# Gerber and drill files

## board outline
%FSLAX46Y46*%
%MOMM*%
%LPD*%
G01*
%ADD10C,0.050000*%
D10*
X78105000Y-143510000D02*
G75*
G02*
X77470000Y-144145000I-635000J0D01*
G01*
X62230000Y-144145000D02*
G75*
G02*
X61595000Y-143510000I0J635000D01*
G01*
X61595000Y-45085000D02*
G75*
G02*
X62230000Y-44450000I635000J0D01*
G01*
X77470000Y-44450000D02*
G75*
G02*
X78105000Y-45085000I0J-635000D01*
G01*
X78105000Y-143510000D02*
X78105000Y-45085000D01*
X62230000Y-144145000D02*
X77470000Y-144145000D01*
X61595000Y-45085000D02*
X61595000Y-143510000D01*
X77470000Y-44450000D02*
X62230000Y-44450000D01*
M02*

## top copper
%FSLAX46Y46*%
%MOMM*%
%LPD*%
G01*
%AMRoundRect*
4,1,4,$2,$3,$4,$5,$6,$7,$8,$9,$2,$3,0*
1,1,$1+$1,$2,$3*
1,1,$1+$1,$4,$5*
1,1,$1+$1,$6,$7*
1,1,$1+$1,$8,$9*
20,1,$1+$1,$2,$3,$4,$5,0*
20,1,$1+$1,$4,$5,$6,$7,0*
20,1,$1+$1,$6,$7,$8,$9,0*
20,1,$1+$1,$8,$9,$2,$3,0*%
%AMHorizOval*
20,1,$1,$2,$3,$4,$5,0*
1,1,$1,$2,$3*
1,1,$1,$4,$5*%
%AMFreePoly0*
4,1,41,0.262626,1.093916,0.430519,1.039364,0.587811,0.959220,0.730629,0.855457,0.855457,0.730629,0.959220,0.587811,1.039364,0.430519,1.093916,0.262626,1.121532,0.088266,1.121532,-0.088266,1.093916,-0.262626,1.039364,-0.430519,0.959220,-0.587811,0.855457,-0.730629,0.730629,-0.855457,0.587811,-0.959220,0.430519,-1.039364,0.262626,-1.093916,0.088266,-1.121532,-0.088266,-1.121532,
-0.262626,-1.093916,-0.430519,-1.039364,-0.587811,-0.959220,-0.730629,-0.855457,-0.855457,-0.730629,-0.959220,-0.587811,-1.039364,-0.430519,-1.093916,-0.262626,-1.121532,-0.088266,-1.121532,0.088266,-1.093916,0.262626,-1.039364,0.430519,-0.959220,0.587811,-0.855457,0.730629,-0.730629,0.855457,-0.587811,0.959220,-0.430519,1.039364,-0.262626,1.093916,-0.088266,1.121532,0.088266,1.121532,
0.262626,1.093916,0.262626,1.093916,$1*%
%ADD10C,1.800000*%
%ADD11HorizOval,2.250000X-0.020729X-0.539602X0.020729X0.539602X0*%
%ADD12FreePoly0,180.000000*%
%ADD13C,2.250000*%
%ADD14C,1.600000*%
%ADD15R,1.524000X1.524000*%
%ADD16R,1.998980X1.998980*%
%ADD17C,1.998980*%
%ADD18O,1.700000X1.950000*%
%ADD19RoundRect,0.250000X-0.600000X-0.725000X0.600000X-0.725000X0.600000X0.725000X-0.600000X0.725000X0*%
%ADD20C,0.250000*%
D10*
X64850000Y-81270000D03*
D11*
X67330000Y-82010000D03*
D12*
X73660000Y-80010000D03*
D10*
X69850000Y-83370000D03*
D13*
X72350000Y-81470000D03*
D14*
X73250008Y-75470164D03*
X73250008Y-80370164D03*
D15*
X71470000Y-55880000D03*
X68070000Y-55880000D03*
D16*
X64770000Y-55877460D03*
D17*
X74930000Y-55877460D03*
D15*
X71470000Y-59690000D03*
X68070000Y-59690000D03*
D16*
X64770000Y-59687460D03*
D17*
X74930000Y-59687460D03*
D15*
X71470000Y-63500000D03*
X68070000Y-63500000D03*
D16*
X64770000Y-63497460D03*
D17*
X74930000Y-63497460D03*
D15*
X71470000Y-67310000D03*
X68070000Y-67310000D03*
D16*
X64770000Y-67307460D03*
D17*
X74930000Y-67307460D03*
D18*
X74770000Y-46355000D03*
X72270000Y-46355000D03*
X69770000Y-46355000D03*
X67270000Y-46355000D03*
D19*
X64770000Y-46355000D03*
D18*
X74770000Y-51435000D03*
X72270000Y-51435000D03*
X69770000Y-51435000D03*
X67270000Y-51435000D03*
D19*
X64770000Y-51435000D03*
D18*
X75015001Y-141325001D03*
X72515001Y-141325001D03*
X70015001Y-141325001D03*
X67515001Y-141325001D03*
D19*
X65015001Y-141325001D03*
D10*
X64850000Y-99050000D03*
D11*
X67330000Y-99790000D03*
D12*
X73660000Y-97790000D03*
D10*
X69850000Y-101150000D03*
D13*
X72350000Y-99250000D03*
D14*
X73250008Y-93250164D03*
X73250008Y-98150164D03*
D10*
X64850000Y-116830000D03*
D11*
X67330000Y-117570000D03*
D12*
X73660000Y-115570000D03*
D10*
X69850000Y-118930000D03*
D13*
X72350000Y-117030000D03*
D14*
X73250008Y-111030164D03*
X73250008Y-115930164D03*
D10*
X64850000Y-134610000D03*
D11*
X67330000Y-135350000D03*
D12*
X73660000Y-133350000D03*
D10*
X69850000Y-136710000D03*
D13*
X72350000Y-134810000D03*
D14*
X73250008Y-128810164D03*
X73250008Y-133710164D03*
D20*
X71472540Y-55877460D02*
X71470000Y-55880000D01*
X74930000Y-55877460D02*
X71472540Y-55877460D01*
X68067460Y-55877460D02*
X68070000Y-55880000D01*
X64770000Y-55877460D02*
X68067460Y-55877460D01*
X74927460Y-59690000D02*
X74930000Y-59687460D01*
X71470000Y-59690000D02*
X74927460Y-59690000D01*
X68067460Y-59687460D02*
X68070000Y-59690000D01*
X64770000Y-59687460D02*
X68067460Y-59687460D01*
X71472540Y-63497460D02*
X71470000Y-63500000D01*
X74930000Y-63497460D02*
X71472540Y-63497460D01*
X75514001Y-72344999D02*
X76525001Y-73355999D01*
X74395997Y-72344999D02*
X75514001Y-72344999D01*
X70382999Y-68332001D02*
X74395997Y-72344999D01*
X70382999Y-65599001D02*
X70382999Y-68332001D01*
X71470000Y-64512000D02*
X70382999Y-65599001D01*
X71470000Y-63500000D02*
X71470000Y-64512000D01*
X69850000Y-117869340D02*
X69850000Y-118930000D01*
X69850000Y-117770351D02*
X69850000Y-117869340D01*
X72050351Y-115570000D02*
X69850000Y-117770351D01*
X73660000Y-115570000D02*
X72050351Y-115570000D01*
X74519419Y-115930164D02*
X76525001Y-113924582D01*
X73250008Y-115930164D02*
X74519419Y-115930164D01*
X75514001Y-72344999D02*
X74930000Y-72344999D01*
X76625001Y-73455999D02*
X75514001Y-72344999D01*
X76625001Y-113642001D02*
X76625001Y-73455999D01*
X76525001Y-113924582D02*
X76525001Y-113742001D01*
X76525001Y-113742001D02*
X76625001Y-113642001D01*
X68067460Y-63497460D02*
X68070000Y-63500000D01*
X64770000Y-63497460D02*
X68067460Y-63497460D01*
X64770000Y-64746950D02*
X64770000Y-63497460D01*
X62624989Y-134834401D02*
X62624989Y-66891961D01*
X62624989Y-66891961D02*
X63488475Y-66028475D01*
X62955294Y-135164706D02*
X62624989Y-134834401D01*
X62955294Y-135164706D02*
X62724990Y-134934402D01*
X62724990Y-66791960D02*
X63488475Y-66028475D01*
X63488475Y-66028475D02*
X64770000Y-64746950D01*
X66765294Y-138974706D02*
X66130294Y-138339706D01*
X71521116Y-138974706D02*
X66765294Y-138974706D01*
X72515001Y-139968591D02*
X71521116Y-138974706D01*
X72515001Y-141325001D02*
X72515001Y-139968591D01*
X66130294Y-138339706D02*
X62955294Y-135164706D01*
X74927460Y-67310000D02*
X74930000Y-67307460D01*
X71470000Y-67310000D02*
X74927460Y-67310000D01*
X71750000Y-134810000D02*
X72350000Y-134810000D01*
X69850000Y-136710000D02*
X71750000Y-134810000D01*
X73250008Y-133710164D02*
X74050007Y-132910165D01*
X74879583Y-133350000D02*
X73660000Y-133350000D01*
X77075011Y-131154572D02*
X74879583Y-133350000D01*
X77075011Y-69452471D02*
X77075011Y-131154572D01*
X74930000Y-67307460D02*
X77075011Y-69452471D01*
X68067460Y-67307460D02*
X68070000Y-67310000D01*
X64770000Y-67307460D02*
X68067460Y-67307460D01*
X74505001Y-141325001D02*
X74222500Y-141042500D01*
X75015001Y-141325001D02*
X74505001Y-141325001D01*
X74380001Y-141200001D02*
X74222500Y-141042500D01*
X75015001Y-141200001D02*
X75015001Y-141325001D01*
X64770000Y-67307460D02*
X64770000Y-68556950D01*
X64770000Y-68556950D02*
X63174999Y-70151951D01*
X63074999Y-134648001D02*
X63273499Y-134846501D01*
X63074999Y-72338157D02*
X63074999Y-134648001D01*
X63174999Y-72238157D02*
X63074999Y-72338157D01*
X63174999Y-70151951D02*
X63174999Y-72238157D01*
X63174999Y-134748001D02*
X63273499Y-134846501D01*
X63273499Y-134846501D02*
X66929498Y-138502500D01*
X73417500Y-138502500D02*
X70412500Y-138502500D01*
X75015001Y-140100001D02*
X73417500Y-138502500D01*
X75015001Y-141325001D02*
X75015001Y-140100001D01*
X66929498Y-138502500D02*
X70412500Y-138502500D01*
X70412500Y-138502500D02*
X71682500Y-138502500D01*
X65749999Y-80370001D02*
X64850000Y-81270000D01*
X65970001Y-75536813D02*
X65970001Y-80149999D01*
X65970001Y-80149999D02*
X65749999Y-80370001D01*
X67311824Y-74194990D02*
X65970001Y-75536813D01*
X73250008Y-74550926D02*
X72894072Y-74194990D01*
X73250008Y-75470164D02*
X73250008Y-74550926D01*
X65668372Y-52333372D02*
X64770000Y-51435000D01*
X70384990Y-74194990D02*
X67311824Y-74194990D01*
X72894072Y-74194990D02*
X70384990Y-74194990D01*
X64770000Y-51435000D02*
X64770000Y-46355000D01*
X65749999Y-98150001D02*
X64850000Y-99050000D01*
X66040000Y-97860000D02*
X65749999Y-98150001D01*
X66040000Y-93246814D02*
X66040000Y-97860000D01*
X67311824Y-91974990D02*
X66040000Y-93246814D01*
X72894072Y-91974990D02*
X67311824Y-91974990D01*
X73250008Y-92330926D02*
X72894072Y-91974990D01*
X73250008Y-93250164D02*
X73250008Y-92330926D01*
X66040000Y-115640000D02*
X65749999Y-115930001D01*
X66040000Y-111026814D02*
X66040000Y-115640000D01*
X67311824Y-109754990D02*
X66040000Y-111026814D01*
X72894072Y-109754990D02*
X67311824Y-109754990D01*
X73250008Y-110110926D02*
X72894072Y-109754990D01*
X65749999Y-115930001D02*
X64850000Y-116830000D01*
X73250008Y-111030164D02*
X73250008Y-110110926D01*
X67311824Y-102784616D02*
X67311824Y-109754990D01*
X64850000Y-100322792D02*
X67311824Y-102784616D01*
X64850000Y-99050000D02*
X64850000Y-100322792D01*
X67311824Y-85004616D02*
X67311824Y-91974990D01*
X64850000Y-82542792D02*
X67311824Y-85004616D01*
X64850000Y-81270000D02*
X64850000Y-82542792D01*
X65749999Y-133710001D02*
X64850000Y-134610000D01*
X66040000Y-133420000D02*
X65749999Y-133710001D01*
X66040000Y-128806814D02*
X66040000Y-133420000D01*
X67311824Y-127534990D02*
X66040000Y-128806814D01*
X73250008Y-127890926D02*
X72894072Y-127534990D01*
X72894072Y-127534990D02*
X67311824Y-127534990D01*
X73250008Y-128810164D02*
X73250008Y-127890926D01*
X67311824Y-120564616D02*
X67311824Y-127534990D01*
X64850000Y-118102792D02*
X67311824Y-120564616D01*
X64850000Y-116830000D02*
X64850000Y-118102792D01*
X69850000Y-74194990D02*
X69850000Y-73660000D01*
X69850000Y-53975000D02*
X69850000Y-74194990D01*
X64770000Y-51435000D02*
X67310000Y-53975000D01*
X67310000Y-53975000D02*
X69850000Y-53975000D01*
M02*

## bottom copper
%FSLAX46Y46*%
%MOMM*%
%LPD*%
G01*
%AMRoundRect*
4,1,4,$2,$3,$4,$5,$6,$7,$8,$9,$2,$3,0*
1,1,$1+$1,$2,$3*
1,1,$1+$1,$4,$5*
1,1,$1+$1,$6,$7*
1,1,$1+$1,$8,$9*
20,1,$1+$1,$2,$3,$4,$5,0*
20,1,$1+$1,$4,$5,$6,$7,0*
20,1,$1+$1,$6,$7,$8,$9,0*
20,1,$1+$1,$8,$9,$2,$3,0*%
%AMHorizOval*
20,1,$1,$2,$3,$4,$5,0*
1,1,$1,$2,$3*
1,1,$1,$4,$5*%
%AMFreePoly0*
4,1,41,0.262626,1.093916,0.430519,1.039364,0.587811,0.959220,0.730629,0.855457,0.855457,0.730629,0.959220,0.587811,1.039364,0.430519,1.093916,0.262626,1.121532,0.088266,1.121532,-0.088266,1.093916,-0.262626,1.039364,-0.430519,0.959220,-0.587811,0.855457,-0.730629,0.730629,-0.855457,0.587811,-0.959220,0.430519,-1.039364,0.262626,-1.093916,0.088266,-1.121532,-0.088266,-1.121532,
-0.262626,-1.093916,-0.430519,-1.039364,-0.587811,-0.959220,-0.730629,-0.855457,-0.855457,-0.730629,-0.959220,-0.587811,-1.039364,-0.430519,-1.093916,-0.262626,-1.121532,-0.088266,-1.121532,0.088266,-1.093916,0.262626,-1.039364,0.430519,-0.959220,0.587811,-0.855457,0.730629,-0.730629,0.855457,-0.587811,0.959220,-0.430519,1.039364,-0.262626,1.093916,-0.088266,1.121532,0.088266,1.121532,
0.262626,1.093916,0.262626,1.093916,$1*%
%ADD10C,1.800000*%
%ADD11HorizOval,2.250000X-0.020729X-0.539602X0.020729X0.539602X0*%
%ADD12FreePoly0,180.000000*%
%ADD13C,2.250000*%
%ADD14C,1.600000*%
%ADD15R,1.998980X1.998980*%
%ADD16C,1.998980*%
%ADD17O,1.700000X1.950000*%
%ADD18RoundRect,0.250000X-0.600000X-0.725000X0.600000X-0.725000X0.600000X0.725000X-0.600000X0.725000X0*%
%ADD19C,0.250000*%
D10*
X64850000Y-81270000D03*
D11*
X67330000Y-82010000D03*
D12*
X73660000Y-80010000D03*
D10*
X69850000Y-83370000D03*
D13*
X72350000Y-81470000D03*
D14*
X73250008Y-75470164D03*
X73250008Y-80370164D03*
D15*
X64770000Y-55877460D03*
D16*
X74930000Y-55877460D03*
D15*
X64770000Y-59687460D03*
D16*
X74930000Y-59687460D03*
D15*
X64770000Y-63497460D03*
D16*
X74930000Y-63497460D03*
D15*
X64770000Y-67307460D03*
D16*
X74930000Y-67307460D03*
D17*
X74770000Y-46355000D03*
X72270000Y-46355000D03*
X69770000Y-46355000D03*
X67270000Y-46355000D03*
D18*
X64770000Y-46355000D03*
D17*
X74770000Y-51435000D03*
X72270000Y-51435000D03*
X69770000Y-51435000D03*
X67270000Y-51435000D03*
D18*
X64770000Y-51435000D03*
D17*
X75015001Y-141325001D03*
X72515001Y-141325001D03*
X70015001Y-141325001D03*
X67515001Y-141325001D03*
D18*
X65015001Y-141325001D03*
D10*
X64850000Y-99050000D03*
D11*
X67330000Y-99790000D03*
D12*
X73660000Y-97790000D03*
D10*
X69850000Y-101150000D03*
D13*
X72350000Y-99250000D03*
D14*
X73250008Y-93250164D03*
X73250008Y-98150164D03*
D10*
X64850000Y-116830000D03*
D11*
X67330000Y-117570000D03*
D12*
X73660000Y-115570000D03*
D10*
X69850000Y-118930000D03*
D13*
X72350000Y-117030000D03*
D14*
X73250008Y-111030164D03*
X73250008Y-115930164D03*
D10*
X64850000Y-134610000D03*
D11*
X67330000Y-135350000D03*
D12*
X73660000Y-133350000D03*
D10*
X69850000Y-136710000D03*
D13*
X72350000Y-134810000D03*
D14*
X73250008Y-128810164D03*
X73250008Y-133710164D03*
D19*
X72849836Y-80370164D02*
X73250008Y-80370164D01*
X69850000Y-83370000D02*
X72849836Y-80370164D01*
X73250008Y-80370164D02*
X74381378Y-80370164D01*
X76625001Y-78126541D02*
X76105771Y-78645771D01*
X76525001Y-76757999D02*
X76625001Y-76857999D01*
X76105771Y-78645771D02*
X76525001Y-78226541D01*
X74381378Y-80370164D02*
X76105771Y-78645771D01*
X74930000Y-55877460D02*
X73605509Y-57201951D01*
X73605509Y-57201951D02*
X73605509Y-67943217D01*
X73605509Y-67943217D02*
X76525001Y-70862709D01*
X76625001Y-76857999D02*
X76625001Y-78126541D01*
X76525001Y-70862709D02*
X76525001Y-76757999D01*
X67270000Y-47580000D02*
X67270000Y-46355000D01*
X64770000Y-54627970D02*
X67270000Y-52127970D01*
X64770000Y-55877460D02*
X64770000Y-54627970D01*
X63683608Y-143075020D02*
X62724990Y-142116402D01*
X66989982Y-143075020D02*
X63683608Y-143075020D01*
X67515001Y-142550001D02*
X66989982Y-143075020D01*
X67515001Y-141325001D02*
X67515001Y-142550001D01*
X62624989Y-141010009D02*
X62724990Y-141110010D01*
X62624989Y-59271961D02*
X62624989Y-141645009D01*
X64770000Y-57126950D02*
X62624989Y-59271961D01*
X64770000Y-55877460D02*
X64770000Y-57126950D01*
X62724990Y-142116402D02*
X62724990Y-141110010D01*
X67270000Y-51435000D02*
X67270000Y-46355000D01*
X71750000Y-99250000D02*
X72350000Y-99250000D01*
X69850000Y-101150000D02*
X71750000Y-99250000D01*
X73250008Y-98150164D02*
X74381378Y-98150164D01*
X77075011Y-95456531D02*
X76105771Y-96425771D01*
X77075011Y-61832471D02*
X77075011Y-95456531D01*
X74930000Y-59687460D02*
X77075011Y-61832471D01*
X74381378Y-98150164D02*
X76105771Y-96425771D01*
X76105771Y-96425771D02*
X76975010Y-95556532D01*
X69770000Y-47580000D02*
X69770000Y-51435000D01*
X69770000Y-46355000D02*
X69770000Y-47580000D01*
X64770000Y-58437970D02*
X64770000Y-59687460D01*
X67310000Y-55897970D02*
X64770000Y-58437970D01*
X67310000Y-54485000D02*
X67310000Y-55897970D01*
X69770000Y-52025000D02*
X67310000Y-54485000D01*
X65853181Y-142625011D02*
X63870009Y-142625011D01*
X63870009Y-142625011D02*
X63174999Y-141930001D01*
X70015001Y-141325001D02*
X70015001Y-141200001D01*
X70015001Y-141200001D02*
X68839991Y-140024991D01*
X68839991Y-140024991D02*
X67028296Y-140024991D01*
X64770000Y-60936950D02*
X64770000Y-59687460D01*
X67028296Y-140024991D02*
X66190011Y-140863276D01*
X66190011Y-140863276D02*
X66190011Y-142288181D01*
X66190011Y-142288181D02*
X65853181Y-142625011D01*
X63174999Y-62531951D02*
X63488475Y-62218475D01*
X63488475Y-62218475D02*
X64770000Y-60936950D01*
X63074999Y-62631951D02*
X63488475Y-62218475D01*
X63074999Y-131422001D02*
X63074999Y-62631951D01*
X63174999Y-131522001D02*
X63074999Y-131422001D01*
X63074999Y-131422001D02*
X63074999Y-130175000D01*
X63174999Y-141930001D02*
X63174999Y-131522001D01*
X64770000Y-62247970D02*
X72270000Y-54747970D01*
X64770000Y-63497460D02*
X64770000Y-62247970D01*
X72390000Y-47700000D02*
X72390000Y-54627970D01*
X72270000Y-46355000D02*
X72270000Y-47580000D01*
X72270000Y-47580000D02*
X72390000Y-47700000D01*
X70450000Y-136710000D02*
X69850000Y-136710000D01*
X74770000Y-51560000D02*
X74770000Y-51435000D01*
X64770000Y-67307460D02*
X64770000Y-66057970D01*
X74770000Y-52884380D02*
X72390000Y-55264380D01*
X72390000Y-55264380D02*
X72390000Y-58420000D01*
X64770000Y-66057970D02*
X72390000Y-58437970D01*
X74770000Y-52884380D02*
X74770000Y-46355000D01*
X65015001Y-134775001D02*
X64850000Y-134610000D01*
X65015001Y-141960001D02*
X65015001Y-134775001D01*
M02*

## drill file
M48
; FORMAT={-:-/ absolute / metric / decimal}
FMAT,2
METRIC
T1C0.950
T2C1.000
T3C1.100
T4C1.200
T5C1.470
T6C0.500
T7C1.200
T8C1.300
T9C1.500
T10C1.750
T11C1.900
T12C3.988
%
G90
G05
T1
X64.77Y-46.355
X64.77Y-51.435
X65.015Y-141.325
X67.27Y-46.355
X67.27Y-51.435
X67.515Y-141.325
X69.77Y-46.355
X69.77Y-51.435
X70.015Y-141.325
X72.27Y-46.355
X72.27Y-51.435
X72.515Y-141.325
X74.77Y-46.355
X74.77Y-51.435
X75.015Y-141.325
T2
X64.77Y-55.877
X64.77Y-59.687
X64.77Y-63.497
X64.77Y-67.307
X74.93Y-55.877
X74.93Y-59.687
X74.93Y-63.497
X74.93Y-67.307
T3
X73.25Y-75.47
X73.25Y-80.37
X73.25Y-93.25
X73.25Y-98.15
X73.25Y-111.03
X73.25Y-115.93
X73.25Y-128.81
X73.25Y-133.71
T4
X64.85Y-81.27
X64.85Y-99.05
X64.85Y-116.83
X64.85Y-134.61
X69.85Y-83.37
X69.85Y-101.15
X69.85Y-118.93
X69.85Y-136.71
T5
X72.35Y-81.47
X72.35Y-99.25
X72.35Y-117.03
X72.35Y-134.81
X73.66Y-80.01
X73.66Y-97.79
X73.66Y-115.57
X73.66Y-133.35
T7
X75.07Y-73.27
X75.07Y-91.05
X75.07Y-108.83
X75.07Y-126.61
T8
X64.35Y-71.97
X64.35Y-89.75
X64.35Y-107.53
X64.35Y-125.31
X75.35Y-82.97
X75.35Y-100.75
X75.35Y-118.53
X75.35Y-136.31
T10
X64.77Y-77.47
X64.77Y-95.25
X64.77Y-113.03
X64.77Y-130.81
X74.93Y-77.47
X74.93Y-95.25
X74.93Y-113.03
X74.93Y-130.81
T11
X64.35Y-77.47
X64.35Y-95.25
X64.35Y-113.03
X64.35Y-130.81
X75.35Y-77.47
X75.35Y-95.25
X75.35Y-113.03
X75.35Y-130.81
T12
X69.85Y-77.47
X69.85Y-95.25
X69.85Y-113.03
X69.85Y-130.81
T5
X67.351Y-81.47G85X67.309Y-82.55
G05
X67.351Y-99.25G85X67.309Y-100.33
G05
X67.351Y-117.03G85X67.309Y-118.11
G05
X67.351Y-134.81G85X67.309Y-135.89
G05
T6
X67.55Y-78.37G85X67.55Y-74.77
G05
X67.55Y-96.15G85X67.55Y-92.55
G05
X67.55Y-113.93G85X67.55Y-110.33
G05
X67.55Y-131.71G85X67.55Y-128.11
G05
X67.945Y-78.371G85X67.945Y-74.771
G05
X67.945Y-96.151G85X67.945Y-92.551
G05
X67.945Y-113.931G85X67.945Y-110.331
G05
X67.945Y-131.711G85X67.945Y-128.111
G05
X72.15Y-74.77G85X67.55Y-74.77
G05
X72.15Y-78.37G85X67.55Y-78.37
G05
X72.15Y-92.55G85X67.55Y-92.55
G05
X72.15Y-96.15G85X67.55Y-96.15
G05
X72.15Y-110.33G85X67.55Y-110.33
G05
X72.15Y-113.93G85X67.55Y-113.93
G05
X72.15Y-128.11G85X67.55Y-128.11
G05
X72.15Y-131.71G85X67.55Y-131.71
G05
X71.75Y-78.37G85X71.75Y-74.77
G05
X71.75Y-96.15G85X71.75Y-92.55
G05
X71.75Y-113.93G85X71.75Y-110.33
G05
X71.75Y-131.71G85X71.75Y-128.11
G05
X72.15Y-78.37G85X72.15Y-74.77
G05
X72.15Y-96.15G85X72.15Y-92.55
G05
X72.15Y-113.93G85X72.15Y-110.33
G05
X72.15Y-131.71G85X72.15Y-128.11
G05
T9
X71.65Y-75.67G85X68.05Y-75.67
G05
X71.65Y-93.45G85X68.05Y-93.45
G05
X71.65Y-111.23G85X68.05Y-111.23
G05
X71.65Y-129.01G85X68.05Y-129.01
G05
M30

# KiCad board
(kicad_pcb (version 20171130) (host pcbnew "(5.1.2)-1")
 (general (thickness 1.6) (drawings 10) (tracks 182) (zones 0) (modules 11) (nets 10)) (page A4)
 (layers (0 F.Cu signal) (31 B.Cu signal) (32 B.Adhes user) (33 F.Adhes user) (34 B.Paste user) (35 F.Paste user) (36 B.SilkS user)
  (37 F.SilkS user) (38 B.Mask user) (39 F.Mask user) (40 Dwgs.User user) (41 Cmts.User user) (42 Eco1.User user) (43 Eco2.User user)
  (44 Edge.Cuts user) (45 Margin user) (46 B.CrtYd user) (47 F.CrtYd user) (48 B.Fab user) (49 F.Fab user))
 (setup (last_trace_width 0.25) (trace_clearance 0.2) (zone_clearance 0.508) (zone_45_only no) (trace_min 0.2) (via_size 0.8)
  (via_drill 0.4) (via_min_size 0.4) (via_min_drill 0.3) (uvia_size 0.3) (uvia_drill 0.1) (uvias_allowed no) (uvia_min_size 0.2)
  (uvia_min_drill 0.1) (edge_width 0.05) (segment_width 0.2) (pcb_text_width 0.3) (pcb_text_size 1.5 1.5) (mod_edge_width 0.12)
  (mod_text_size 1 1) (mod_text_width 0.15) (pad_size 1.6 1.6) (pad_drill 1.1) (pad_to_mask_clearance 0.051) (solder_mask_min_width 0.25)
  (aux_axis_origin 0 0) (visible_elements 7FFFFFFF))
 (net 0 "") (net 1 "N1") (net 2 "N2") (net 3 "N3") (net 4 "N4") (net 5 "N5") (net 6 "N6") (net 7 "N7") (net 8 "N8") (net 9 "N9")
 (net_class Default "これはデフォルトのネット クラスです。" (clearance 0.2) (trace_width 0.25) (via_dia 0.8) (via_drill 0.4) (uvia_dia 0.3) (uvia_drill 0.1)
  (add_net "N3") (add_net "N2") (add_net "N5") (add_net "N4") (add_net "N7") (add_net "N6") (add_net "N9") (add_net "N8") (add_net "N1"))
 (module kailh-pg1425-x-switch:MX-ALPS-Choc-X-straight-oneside (layer F.Cu) (at 67.31 82.55 180)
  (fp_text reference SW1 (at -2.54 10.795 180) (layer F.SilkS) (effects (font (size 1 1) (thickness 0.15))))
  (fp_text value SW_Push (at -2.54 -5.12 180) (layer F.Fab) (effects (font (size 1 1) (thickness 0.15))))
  (pad "" np_thru_hole circle (at 2.96 5.08 228.1) (size 1.9 1.9) (drill 1.9) (layers *.Cu *.Mask))
  (pad "" np_thru_hole circle (at -8.04 5.08 228.1) (size 1.9 1.9) (drill 1.9) (layers *.Cu *.Mask))
  (pad 1 thru_hole circle (at 2.46 1.28 180) (size 1.8 1.8) (drill 1.2) (layers *.Cu *.Mask) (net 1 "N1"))
  (pad "" np_thru_hole circle (at 2.54 5.08 228.0996) (size 1.75 1.75) (drill 1.75) (layers *.Cu *.Mask))
  (pad "" np_thru_hole circle (at -7.62 5.08 228.0996) (size 1.75 1.75) (drill 1.75) (layers *.Cu *.Mask))
  (pad "" np_thru_hole circle (at -2.54 5.08 180) (size 3.9878 3.9878) (drill 3.9878) (layers *.Cu *.Mask))
  (pad 3 thru_hole oval (at -0.02 0.54 267.8) (size 3.33 2.25) (drill oval 2.55 1.47) (layers *.Cu *.Mask))
  (pad 2 thru_hole custom (at -6.35 2.54 180) (size 2.25 2.25) (drill 1.47) (layers *.Cu *.Mask) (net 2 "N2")
   (options (clearance outline) (anchor circle)) (primitives))
  (pad "" np_thru_hole circle (at -7.76 9.28 228.1) (size 1.2 1.2) (drill 1.2) (layers *.Cu *.Mask))
  (pad "" np_thru_hole oval (at -0.635 5.97916 180) (size 0.5 4.1) (drill oval 0.5 4.1) (layers *.Cu *.Mask))
  (pad "" np_thru_hole oval (at -4.84 5.98 180) (size 0.5 4.1) (drill oval 0.5 4.1) (layers *.Cu *.Mask))
  (pad "" np_thru_hole oval (at -2.54 6.88 180) (size 5.1 1.5) (drill oval 5.1 1.5) (layers *.Cu *.Mask))
  (pad "" np_thru_hole oval (at -4.44 5.98 180) (size 0.5 4.1) (drill oval 0.5 4.1) (layers *.Cu *.Mask))
  (pad "" np_thru_hole oval (at -2.54 7.78 180) (size 5.1 0.5) (drill oval 5.1 0.5) (layers *.Cu *.Mask))
  (pad "" np_thru_hole oval (at -2.54 4.18 180) (size 5.1 0.5) (drill oval 5.1 0.5) (layers *.Cu *.Mask))
  (pad "" np_thru_hole oval (at -0.24 5.98 180) (size 0.5 4.1) (drill oval 0.5 4.1) (layers *.Cu *.Mask))
  (pad 2 thru_hole circle (at -2.54 -0.82 180) (size 1.8 1.8) (drill 1.2) (layers *.Cu *.Mask) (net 2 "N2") (zone_connect 0))
  (pad 2 thru_hole circle (at -5.04 1.08 180) (size 2.25 2.25) (drill 1.47) (layers *.Cu B.Mask) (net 2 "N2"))
  (pad "" np_thru_hole circle (at 2.959992 10.579836) (size 1.3 1.3) (drill 1.3) (layers *.Cu *.Mask))
  (pad 1 thru_hole circle (at -5.940008 7.079836) (size 1.6 1.6) (drill 1.1) (layers *.Cu *.Mask) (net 1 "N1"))
  (pad "" np_thru_hole circle (at -8.040008 -0.420164) (size 1.3 1.3) (drill 1.3) (layers *.Cu *.Mask))
  (pad 2 thru_hole circle (at -5.940008 2.179836) (size 1.6 1.6) (drill 1.1) (layers *.Cu *.Mask) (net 2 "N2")))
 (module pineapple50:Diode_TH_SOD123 (layer F.Cu) (at 64.77 55.88)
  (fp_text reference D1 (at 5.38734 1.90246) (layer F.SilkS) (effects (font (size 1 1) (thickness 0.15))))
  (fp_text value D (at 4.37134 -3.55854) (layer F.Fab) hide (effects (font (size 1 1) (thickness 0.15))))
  (pad 2 smd rect (at 6.7 0) (size 1.524 1.524) (layers F.Cu F.Paste F.Mask) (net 2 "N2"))
  (pad 1 smd rect (at 3.3 0) (size 1.524 1.524) (layers F.Cu F.Paste F.Mask) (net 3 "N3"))
  (pad 1 thru_hole rect (at 0 -0.00254 180) (size 1.99898 1.99898) (drill 1) (layers *.Cu *.Mask) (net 3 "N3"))
  (pad 2 thru_hole circle (at 10.16 -0.00254 180) (size 1.99898 1.99898) (drill 1) (layers *.Cu *.Mask) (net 2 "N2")))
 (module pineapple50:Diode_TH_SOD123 (layer F.Cu) (at 64.77 59.69)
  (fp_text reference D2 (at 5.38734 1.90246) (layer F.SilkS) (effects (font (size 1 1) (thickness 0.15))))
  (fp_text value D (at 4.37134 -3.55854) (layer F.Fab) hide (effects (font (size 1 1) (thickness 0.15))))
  (pad 2 smd rect (at 6.7 0) (size 1.524 1.524) (layers F.Cu F.Paste F.Mask) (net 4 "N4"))
  (pad 1 smd rect (at 3.3 0) (size 1.524 1.524) (layers F.Cu F.Paste F.Mask) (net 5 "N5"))
  (pad 1 thru_hole rect (at 0 -0.00254 180) (size 1.99898 1.99898) (drill 1) (layers *.Cu *.Mask) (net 5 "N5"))
  (pad 2 thru_hole circle (at 10.16 -0.00254 180) (size 1.99898 1.99898) (drill 1) (layers *.Cu *.Mask) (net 4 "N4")))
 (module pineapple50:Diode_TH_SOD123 (layer F.Cu) (at 64.77 63.5)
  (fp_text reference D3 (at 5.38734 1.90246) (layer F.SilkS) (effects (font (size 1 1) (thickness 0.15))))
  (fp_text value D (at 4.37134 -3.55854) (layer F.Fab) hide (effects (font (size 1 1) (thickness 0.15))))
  (pad 2 smd rect (at 6.7 0) (size 1.524 1.524) (layers F.Cu F.Paste F.Mask) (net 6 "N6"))
  (pad 1 smd rect (at 3.3 0) (size 1.524 1.524) (layers F.Cu F.Paste F.Mask) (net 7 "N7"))
  (pad 1 thru_hole rect (at 0 -0.00254 180) (size 1.99898 1.99898) (drill 1) (layers *.Cu *.Mask) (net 7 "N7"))
  (pad 2 thru_hole circle (at 10.16 -0.00254 180) (size 1.99898 1.99898) (drill 1) (layers *.Cu *.Mask) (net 6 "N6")))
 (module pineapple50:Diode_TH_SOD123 (layer F.Cu) (at 64.77 67.31)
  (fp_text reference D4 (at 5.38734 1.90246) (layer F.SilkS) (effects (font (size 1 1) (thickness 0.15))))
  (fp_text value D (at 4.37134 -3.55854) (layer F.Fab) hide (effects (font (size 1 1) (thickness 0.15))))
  (pad 2 smd rect (at 6.7 0) (size 1.524 1.524) (layers F.Cu F.Paste F.Mask) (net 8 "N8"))
  (pad 1 smd rect (at 3.3 0) (size 1.524 1.524) (layers F.Cu F.Paste F.Mask) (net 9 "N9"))
  (pad 1 thru_hole rect (at 0 -0.00254 180) (size 1.99898 1.99898) (drill 1) (layers *.Cu *.Mask) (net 9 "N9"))
  (pad 2 thru_hole circle (at 10.16 -0.00254 180) (size 1.99898 1.99898) (drill 1) (layers *.Cu *.Mask) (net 8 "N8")))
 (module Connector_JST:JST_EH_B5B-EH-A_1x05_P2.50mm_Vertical (layer F.Cu) (at 64.77 46.355)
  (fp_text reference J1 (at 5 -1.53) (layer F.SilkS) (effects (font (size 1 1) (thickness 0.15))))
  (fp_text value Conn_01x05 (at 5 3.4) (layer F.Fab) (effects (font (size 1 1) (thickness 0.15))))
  (pad 5 thru_hole oval (at 10 0) (size 1.7 1.95) (drill 0.95) (layers *.Cu *.Mask) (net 9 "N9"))
  (pad 4 thru_hole oval (at 7.5 0) (size 1.7 1.95) (drill 0.95) (layers *.Cu *.Mask) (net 7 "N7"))
  (pad 3 thru_hole oval (at 5 0) (size 1.7 1.95) (drill 0.95) (layers *.Cu *.Mask) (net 5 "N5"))
  (pad 2 thru_hole oval (at 2.5 0) (size 1.7 1.95) (drill 0.95) (layers *.Cu *.Mask) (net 3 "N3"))
  (pad 1 thru_hole roundrect (at 0 0) (size 1.7 1.95) (drill 0.95) (layers *.Cu *.Mask) (roundrect_rratio 0.147059) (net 1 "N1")))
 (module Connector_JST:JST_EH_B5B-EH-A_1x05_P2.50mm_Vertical (layer F.Cu) (at 64.77 51.435)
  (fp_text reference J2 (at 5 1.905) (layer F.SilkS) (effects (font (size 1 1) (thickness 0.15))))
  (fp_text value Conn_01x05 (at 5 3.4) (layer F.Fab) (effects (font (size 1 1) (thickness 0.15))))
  (pad 5 thru_hole oval (at 10 0) (size 1.7 1.95) (drill 0.95) (layers *.Cu *.Mask) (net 9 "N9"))
  (pad 4 thru_hole oval (at 7.5 0) (size 1.7 1.95) (drill 0.95) (layers *.Cu *.Mask) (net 7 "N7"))
  (pad 3 thru_hole oval (at 5 0) (size 1.7 1.95) (drill 0.95) (layers *.Cu *.Mask) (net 5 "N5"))
  (pad 2 thru_hole oval (at 2.5 0) (size 1.7 1.95) (drill 0.95) (layers *.Cu *.Mask) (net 3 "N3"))
  (pad 1 thru_hole roundrect (at 0 0) (size 1.7 1.95) (drill 0.95) (layers *.Cu *.Mask) (roundrect_rratio 0.147059) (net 1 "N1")))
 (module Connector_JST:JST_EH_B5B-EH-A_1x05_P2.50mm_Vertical (layer F.Cu) (at 65.015001 141.325001)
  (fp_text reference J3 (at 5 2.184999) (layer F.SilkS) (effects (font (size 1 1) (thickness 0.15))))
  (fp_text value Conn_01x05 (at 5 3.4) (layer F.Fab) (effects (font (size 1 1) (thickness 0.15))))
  (pad 5 thru_hole oval (at 10 0) (size 1.7 1.95) (drill 0.95) (layers *.Cu *.Mask) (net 9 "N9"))
  (pad 4 thru_hole oval (at 7.5 0) (size 1.7 1.95) (drill 0.95) (layers *.Cu *.Mask) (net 7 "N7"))
  (pad 3 thru_hole oval (at 5 0) (size 1.7 1.95) (drill 0.95) (layers *.Cu *.Mask) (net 5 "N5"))
  (pad 2 thru_hole oval (at 2.5 0) (size 1.7 1.95) (drill 0.95) (layers *.Cu *.Mask) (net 3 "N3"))
  (pad 1 thru_hole roundrect (at 0 0) (size 1.7 1.95) (drill 0.95) (layers *.Cu *.Mask) (roundrect_rratio 0.147059) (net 1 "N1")))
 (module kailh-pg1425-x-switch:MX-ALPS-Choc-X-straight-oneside (layer F.Cu) (at 67.31 100.33 180)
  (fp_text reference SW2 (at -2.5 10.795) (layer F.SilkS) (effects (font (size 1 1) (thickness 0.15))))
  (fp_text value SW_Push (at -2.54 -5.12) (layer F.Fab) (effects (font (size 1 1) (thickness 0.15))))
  (pad "" np_thru_hole circle (at 2.96 5.08 228.1) (size 1.9 1.9) (drill 1.9) (layers *.Cu *.Mask))
  (pad "" np_thru_hole circle (at -8.04 5.08 228.1) (size 1.9 1.9) (drill 1.9) (layers *.Cu *.Mask))
  (pad 1 thru_hole circle (at 2.46 1.28 180) (size 1.8 1.8) (drill 1.2) (layers *.Cu *.Mask) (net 1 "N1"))
  (pad "" np_thru_hole circle (at 2.54 5.08 228.0996) (size 1.75 1.75) (drill 1.75) (layers *.Cu *.Mask))
  (pad "" np_thru_hole circle (at -7.62 5.08 228.0996) (size 1.75 1.75) (drill 1.75) (layers *.Cu *.Mask))
  (pad "" np_thru_hole circle (at -2.54 5.08 180) (size 3.9878 3.9878) (drill 3.9878) (layers *.Cu *.Mask))
  (pad 3 thru_hole oval (at -0.02 0.54 267.8) (size 3.33 2.25) (drill oval 2.55 1.47) (layers *.Cu *.Mask))
  (pad 2 thru_hole custom (at -6.35 2.54 180) (size 2.25 2.25) (drill 1.47) (layers *.Cu *.Mask) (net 4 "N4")
   (options (clearance outline) (anchor circle)) (primitives))
  (pad "" np_thru_hole circle (at -7.76 9.28 228.1) (size 1.2 1.2) (drill 1.2) (layers *.Cu *.Mask))
  (pad "" np_thru_hole oval (at -0.635 5.97916 180) (size 0.5 4.1) (drill oval 0.5 4.1) (layers *.Cu *.Mask))
  (pad "" np_thru_hole oval (at -4.84 5.98 180) (size 0.5 4.1) (drill oval 0.5 4.1) (layers *.Cu *.Mask))
  (pad "" np_thru_hole oval (at -2.54 6.88 180) (size 5.1 1.5) (drill oval 5.1 1.5) (layers *.Cu *.Mask))
  (pad "" np_thru_hole oval (at -4.44 5.98 180) (size 0.5 4.1) (drill oval 0.5 4.1) (layers *.Cu *.Mask))
  (pad "" np_thru_hole oval (at -2.54 7.78 180) (size 5.1 0.5) (drill oval 5.1 0.5) (layers *.Cu *.Mask))
  (pad "" np_thru_hole oval (at -2.54 4.18 180) (size 5.1 0.5) (drill oval 5.1 0.5) (layers *.Cu *.Mask))
  (pad "" np_thru_hole oval (at -0.24 5.98 180) (size 0.5 4.1) (drill oval 0.5 4.1) (layers *.Cu *.Mask))
  (pad 2 thru_hole circle (at -2.54 -0.82 180) (size 1.8 1.8) (drill 1.2) (layers *.Cu *.Mask) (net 4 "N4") (zone_connect 0))
  (pad 2 thru_hole circle (at -5.04 1.08 180) (size 2.25 2.25) (drill 1.47) (layers *.Cu B.Mask) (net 4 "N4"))
  (pad "" np_thru_hole circle (at 2.959992 10.579836) (size 1.3 1.3) (drill 1.3) (layers *.Cu *.Mask))
  (pad 1 thru_hole circle (at -5.940008 7.079836) (size 1.6 1.6) (drill 1.1) (layers *.Cu *.Mask) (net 1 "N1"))
  (pad "" np_thru_hole circle (at -8.040008 -0.420164) (size 1.3 1.3) (drill 1.3) (layers *.Cu *.Mask))
  (pad 2 thru_hole circle (at -5.940008 2.179836) (size 1.6 1.6) (drill 1.1) (layers *.Cu *.Mask) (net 4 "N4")))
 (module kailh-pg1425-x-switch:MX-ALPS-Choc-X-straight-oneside (layer F.Cu) (at 67.31 118.11 180)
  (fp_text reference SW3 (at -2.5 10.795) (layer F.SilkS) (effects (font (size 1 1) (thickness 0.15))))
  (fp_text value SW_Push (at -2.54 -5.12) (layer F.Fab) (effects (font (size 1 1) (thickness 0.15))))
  (pad "" np_thru_hole circle (at 2.96 5.08 228.1) (size 1.9 1.9) (drill 1.9) (layers *.Cu *.Mask))
  (pad "" np_thru_hole circle (at -8.04 5.08 228.1) (size 1.9 1.9) (drill 1.9) (layers *.Cu *.Mask))
  (pad 1 thru_hole circle (at 2.46 1.28 180) (size 1.8 1.8) (drill 1.2) (layers *.Cu *.Mask) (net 1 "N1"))
  (pad "" np_thru_hole circle (at 2.54 5.08 228.0996) (size 1.75 1.75) (drill 1.75) (layers *.Cu *.Mask))
  (pad "" np_thru_hole circle (at -7.62 5.08 228.0996) (size 1.75 1.75) (drill 1.75) (layers *.Cu *.Mask))
  (pad "" np_thru_hole circle (at -2.54 5.08 180) (size 3.9878 3.9878) (drill 3.9878) (layers *.Cu *.Mask))
  (pad 3 thru_hole oval (at -0.02 0.54 267.8) (size 3.33 2.25) (drill oval 2.55 1.47) (layers *.Cu *.Mask))
  (pad 2 thru_hole custom (at -6.35 2.54 180) (size 2.25 2.25) (drill 1.47) (layers *.Cu *.Mask) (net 6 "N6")
   (options (clearance outline) (anchor circle)) (primitives))
  (pad "" np_thru_hole circle (at -7.76 9.28 228.1) (size 1.2 1.2) (drill 1.2) (layers *.Cu *.Mask))
  (pad "" np_thru_hole oval (at -0.635 5.97916 180) (size 0.5 4.1) (drill oval 0.5 4.1) (layers *.Cu *.Mask))
  (pad "" np_thru_hole oval (at -4.84 5.98 180) (size 0.5 4.1) (drill oval 0.5 4.1) (layers *.Cu *.Mask))
  (pad "" np_thru_hole oval (at -2.54 6.88 180) (size 5.1 1.5) (drill oval 5.1 1.5) (layers *.Cu *.Mask))
  (pad "" np_thru_hole oval (at -4.44 5.98 180) (size 0.5 4.1) (drill oval 0.5 4.1) (layers *.Cu *.Mask))
  (pad "" np_thru_hole oval (at -2.54 7.78 180) (size 5.1 0.5) (drill oval 5.1 0.5) (layers *.Cu *.Mask))
  (pad "" np_thru_hole oval (at -2.54 4.18 180) (size 5.1 0.5) (drill oval 5.1 0.5) (layers *.Cu *.Mask))
  (pad "" np_thru_hole oval (at -0.24 5.98 180) (size 0.5 4.1) (drill oval 0.5 4.1) (layers *.Cu *.Mask))
  (pad 2 thru_hole circle (at -2.54 -0.82 180) (size 1.8 1.8) (drill 1.2) (layers *.Cu *.Mask) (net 6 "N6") (zone_connect 0))
  (pad 2 thru_hole circle (at -5.04 1.08 180) (size 2.25 2.25) (drill 1.47) (layers *.Cu B.Mask) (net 6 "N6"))
  (pad "" np_thru_hole circle (at 2.959992 10.579836) (size 1.3 1.3) (drill 1.3) (layers *.Cu *.Mask))
  (pad 1 thru_hole circle (at -5.940008 7.079836) (size 1.6 1.6) (drill 1.1) (layers *.Cu *.Mask) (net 1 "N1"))
  (pad "" np_thru_hole circle (at -8.040008 -0.420164) (size 1.3 1.3) (drill 1.3) (layers *.Cu *.Mask))
  (pad 2 thru_hole circle (at -5.940008 2.179836) (size 1.6 1.6) (drill 1.1) (layers *.Cu *.Mask) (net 6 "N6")))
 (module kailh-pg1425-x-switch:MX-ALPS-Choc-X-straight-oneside (layer F.Cu) (at 67.31 135.89 180)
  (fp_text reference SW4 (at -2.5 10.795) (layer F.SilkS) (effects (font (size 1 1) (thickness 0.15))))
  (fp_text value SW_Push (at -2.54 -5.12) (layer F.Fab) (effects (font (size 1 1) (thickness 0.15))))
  (pad "" np_thru_hole circle (at 2.96 5.08 228.1) (size 1.9 1.9) (drill 1.9) (layers *.Cu *.Mask))
  (pad "" np_thru_hole circle (at -8.04 5.08 228.1) (size 1.9 1.9) (drill 1.9) (layers *.Cu *.Mask))
  (pad 1 thru_hole circle (at 2.46 1.28 180) (size 1.8 1.8) (drill 1.2) (layers *.Cu *.Mask) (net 1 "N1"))
  (pad "" np_thru_hole circle (at 2.54 5.08 228.0996) (size 1.75 1.75) (drill 1.75) (layers *.Cu *.Mask))
  (pad "" np_thru_hole circle (at -7.62 5.08 228.0996) (size 1.75 1.75) (drill 1.75) (layers *.Cu *.Mask))
  (pad "" np_thru_hole circle (at -2.54 5.08 180) (size 3.9878 3.9878) (drill 3.9878) (layers *.Cu *.Mask))
  (pad 3 thru_hole oval (at -0.02 0.54 267.8) (size 3.33 2.25) (drill oval 2.55 1.47) (layers *.Cu *.Mask))
  (pad 2 thru_hole custom (at -6.35 2.54 180) (size 2.25 2.25) (drill 1.47) (layers *.Cu *.Mask) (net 8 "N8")
   (options (clearance outline) (anchor circle)) (primitives))
  (pad "" np_thru_hole circle (at -7.76 9.28 228.1) (size 1.2 1.2) (drill 1.2) (layers *.Cu *.Mask))
  (pad "" np_thru_hole oval (at -0.635 5.97916 180) (size 0.5 4.1) (drill oval 0.5 4.1) (layers *.Cu *.Mask))
  (pad "" np_thru_hole oval (at -4.84 5.98 180) (size 0.5 4.1) (drill oval 0.5 4.1) (layers *.Cu *.Mask))
  (pad "" np_thru_hole oval (at -2.54 6.88 180) (size 5.1 1.5) (drill oval 5.1 1.5) (layers *.Cu *.Mask))
  (pad "" np_thru_hole oval (at -4.44 5.98 180) (size 0.5 4.1) (drill oval 0.5 4.1) (layers *.Cu *.Mask))
  (pad "" np_thru_hole oval (at -2.54 7.78 180) (size 5.1 0.5) (drill oval 5.1 0.5) (layers *.Cu *.Mask))
  (pad "" np_thru_hole oval (at -2.54 4.18 180) (size 5.1 0.5) (drill oval 5.1 0.5) (layers *.Cu *.Mask))
  (pad "" np_thru_hole oval (at -0.24 5.98 180) (size 0.5 4.1) (drill oval 0.5 4.1) (layers *.Cu *.Mask))
  (pad 2 thru_hole circle (at -2.54 -0.82 180) (size 1.8 1.8) (drill 1.2) (layers *.Cu *.Mask) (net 8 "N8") (zone_connect 0))
  (pad 2 thru_hole circle (at -5.04 1.08 180) (size 2.25 2.25) (drill 1.47) (layers *.Cu B.Mask) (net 8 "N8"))
  (pad "" np_thru_hole circle (at 2.959992 10.579836) (size 1.3 1.3) (drill 1.3) (layers *.Cu *.Mask))
  (pad 1 thru_hole circle (at -5.940008 7.079836) (size 1.6 1.6) (drill 1.1) (layers *.Cu *.Mask) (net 1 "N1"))
  (pad "" np_thru_hole circle (at -8.040008 -0.420164) (size 1.3 1.3) (drill 1.3) (layers *.Cu *.Mask))
  (pad 2 thru_hole circle (at -5.940008 2.179836) (size 1.6 1.6) (drill 1.1) (layers *.Cu *.Mask) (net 8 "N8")))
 (gr_arc (start 77.47 143.51) (end 77.47 144.145) (angle -90) (layer Edge.Cuts) (width 0.05))
 (gr_arc (start 62.23 143.51) (end 61.595 143.51) (angle -90) (layer Edge.Cuts) (width 0.05))
 (gr_arc (start 62.23 45.085) (end 62.23 44.45) (angle -90) (layer Edge.Cuts) (width 0.05))
 (gr_arc (start 77.47 45.085) (end 78.105 45.085) (angle -90) (layer Edge.Cuts) (width 0.05))
 (gr_line (start 78.105 143.51) (end 78.105 45.085) (layer Edge.Cuts) (width 0.05))
 (gr_line (start 62.23 144.145) (end 77.47 144.145) (layer Edge.Cuts) (width 0.05))
 (gr_line (start 61.595 45.085) (end 61.595 143.51) (layer Edge.Cuts) (width 0.05))
 (gr_line (start 77.47 44.45) (end 62.23 44.45) (layer Edge.Cuts) (width 0.05))
 (segment (start 72.849836 80.370164) (end 73.250008 80.370164) (width 0.25) (layer B.Cu) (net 2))
 (segment (start 69.85 83.37) (end 72.849836 80.370164) (width 0.25) (layer B.Cu) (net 2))
 (segment (start 73.250008 80.370164) (end 74.381378 80.370164) (width 0.25) (layer B.Cu) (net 2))
 (segment (start 71.47254 55.87746) (end 71.47 55.88) (width 0.25) (layer F.Cu) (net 2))
 (segment (start 74.93 55.87746) (end 71.47254 55.87746) (width 0.25) (layer F.Cu) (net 2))
 (segment (start 76.625001 78.126541) (end 76.105771 78.645771) (width 0.25) (layer B.Cu) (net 2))
 (segment (start 76.525001 76.757999) (end 76.625001 76.857999) (width 0.25) (layer B.Cu) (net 2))
 (segment (start 76.105771 78.645771) (end 76.525001 78.226541) (width 0.25) (layer B.Cu) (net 2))
 (segment (start 74.381378 80.370164) (end 76.105771 78.645771) (width 0.25) (layer B.Cu) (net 2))
 (segment (start 74.93 55.87746) (end 73.605509 57.201951) (width 0.25) (layer B.Cu) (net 2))
 (segment (start 73.605509 57.201951) (end 73.605509 67.943217) (width 0.25) (layer B.Cu) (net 2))
 (segment (start 73.605509 67.943217) (end 76.525001 70.862709) (width 0.25) (layer B.Cu) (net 2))
 (segment (start 76.625001 76.857999) (end 76.625001 78.126541) (width 0.25) (layer B.Cu) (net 2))
 (segment (start 76.525001 70.862709) (end 76.525001 76.757999) (width 0.25) (layer B.Cu) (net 2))
 (segment (start 68.06746 55.87746) (end 68.07 55.88) (width 0.25) (layer F.Cu) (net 3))
 (segment (start 64.77 55.87746) (end 68.06746 55.87746) (width 0.25) (layer F.Cu) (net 3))
 (segment (start 67.27 47.58) (end 67.27 46.355) (width 0.25) (layer B.Cu) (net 3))
 (segment (start 64.77 54.62797) (end 67.27 52.12797) (width 0.25) (layer B.Cu) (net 3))
 (segment (start 64.77 55.87746) (end 64.77 54.62797) (width 0.25) (layer B.Cu) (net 3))
 (segment (start 63.683608 143.07502) (end 62.72499 142.116402) (width 0.25) (layer B.Cu) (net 3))
 (segment (start 66.989982 143.07502) (end 63.683608 143.07502) (width 0.25) (layer B.Cu) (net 3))
 (segment (start 67.515001 142.550001) (end 66.989982 143.07502) (width 0.25) (layer B.Cu) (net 3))
 (segment (start 67.515001 141.325001) (end 67.515001 142.550001) (width 0.25) (layer B.Cu) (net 3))
 (segment (start 62.624989 141.010009) (end 62.72499 141.11001) (width 0.25) (layer B.Cu) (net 3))
 (segment (start 62.624989 59.271961) (end 62.624989 141.645009) (width 0.25) (layer B.Cu) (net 3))
 (segment (start 64.77 57.12695) (end 62.624989 59.271961) (width 0.25) (layer B.Cu) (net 3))
 (segment (start 64.77 55.87746) (end 64.77 57.12695) (width 0.25) (layer B.Cu) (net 3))
 (segment (start 62.72499 142.116402) (end 62.72499 141.11001) (width 0.25) (layer B.Cu) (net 3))
 (segment (start 67.27 51.435) (end 67.27 46.355) (width 0.25) (layer B.Cu) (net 3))
 (segment (start 74.92746 59.69) (end 74.93 59.68746) (width 0.25) (layer F.Cu) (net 4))
 (segment (start 71.47 59.69) (end 74.92746 59.69) (width 0.25) (layer F.Cu) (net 4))
 (segment (start 71.75 99.25) (end 72.35 99.25) (width 0.25) (layer B.Cu) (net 4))
 (segment (start 69.85 101.15) (end 71.75 99.25) (width 0.25) (layer B.Cu) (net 4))
 (segment (start 73.250008 98.150164) (end 74.381378 98.150164) (width 0.25) (layer B.Cu) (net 4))
 (segment (start 77.075011 95.456531) (end 76.105771 96.425771) (width 0.25) (layer B.Cu) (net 4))
 (segment (start 77.075011 61.832471) (end 77.075011 95.456531) (width 0.25) (layer B.Cu) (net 4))
 (segment (start 74.93 59.68746) (end 77.075011 61.832471) (width 0.25) (layer B.Cu) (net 4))
 (segment (start 74.381378 98.150164) (end 76.105771 96.425771) (width 0.25) (layer B.Cu) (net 4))
 (segment (start 76.105771 96.425771) (end 76.97501 95.556532) (width 0.25) (layer B.Cu) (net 4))
 (segment (start 68.06746 59.68746) (end 68.07 59.69) (width 0.25) (layer F.Cu) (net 5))
 (segment (start 64.77 59.68746) (end 68.06746 59.68746) (width 0.25) (layer F.Cu) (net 5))
 (segment (start 69.77 47.58) (end 69.77 51.435) (width 0.25) (layer B.Cu) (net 5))
 (segment (start 69.77 46.355) (end 69.77 47.58) (width 0.25) (layer B.Cu) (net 5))
 (segment (start 64.77 58.43797) (end 64.77 59.68746) (width 0.25) (layer B.Cu) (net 5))
 (segment (start 67.31 55.89797) (end 64.77 58.43797) (width 0.25) (layer B.Cu) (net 5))
 (segment (start 67.31 54.485) (end 67.31 55.89797) (width 0.25) (layer B.Cu) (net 5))
 (segment (start 69.77 52.025) (end 67.31 54.485) (width 0.25) (layer B.Cu) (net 5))
 (segment (start 65.853181 142.625011) (end 63.870009 142.625011) (width 0.25) (layer B.Cu) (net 5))
 (segment (start 63.870009 142.625011) (end 63.174999 141.930001) (width 0.25) (layer B.Cu) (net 5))
 (segment (start 70.015001 141.325001) (end 70.015001 141.200001) (width 0.25) (layer B.Cu) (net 5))
 (segment (start 70.015001 141.200001) (end 68.839991 140.024991) (width 0.25) (layer B.Cu) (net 5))
 (segment (start 68.839991 140.024991) (end 67.028296 140.024991) (width 0.25) (layer B.Cu) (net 5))
 (segment (start 64.77 60.93695) (end 64.77 59.68746) (width 0.25) (layer B.Cu) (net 5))
 (segment (start 67.028296 140.024991) (end 66.190011 140.863276) (width 0.25) (layer B.Cu) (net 5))
 (segment (start 66.190011 140.863276) (end 66.190011 142.288181) (width 0.25) (layer B.Cu) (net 5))
 (segment (start 66.190011 142.288181) (end 65.853181 142.625011) (width 0.25) (layer B.Cu) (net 5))
 (segment (start 63.174999 62.531951) (end 63.488475 62.218475) (width 0.25) (layer B.Cu) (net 5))
 (segment (start 63.488475 62.218475) (end 64.77 60.93695) (width 0.25) (layer B.Cu) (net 5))
 (segment (start 63.074999 62.631951) (end 63.488475 62.218475) (width 0.25) (layer B.Cu) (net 5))
 (segment (start 63.074999 131.422001) (end 63.074999 62.631951) (width 0.25) (layer B.Cu) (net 5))
 (segment (start 63.174999 131.522001) (end 63.074999 131.422001) (width 0.25) (layer B.Cu) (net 5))
 (segment (start 63.074999 131.422001) (end 63.074999 130.175) (width 0.25) (layer B.Cu) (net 5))
 (segment (start 63.174999 141.930001) (end 63.174999 131.522001) (width 0.25) (layer B.Cu) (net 5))
 (segment (start 71.47254 63.49746) (end 71.47 63.5) (width 0.25) (layer F.Cu) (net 6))
 (segment (start 74.93 63.49746) (end 71.47254 63.49746) (width 0.25) (layer F.Cu) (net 6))
 (segment (start 75.514001 72.344999) (end 76.525001 73.355999) (width 0.25) (layer F.Cu) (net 6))
 (segment (start 74.395997 72.344999) (end 75.514001 72.344999) (width 0.25) (layer F.Cu) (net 6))
 (segment (start 70.382999 68.332001) (end 74.395997 72.344999) (width 0.25) (layer F.Cu) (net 6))
 (segment (start 70.382999 65.599001) (end 70.382999 68.332001) (width 0.25) (layer F.Cu) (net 6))
 (segment (start 71.47 64.512) (end 70.382999 65.599001) (width 0.25) (layer F.Cu) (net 6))
 (segment (start 71.47 63.5) (end 71.47 64.512) (width 0.25) (layer F.Cu) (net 6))
 (segment (start 69.85 117.86934) (end 69.85 118.93) (width 0.25) (layer F.Cu) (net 6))
 (segment (start 69.85 117.770351) (end 69.85 117.86934) (width 0.25) (layer F.Cu) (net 6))
 (segment (start 72.050351 115.57) (end 69.85 117.770351) (width 0.25) (layer F.Cu) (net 6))
 (segment (start 73.66 115.57) (end 72.050351 115.57) (width 0.25) (layer F.Cu) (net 6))
 (segment (start 74.519419 115.930164) (end 76.525001 113.924582) (width 0.25) (layer F.Cu) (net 6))
 (segment (start 73.250008 115.930164) (end 74.519419 115.930164) (width 0.25) (layer F.Cu) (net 6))
 (segment (start 75.514001 72.344999) (end 74.93 72.344999) (width 0.25) (layer F.Cu) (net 6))
 (segment (start 76.625001 73.455999) (end 75.514001 72.344999) (width 0.25) (layer F.Cu) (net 6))
 (segment (start 76.625001 113.642001) (end 76.625001 73.455999) (width 0.25) (layer F.Cu) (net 6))
 (segment (start 76.525001 113.924582) (end 76.525001 113.742001) (width 0.25) (layer F.Cu) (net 6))
 (segment (start 76.525001 113.742001) (end 76.625001 113.642001) (width 0.25) (layer F.Cu) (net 6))
 (segment (start 68.06746 63.49746) (end 68.07 63.5) (width 0.25) (layer F.Cu) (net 7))
 (segment (start 64.77 63.49746) (end 68.06746 63.49746) (width 0.25) (layer F.Cu) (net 7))
 (segment (start 64.77 62.24797) (end 72.27 54.74797) (width 0.25) (layer B.Cu) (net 7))
 (segment (start 64.77 63.49746) (end 64.77 62.24797) (width 0.25) (layer B.Cu) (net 7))
 (segment (start 64.77 64.74695) (end 64.77 63.49746) (width 0.25) (layer F.Cu) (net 7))
 (segment (start 62.624989 134.834401) (end 62.624989 66.891961) (width 0.25) (layer F.Cu) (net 7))
 (segment (start 62.624989 66.891961) (end 63.488475 66.028475) (width 0.25) (layer F.Cu) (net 7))
 (segment (start 62.955294 135.164706) (end 62.624989 134.834401) (width 0.25) (layer F.Cu) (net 7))
 (segment (start 62.955294 135.164706) (end 62.72499 134.934402) (width 0.25) (layer F.Cu) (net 7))
 (segment (start 62.72499 66.79196) (end 63.488475 66.028475) (width 0.25) (layer F.Cu) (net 7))
 (segment (start 63.488475 66.028475) (end 64.77 64.74695) (width 0.25) (layer F.Cu) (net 7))
 (segment (start 66.765294 138.974706) (end 66.130294 138.339706) (width 0.25) (layer F.Cu) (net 7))
 (segment (start 71.521116 138.974706) (end 66.765294 138.974706) (width 0.25) (layer F.Cu) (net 7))
 (segment (start 72.515001 139.968591) (end 71.521116 138.974706) (width 0.25) (layer F.Cu) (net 7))
 (segment (start 72.515001 141.325001) (end 72.515001 139.968591) (width 0.25) (layer F.Cu) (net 7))
 (segment (start 66.130294 138.339706) (end 62.955294 135.164706) (width 0.25) (layer F.Cu) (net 7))
 (segment (start 72.39 47.7) (end 72.39 54.62797) (width 0.25) (layer B.Cu) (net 7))
 (segment (start 72.27 46.355) (end 72.27 47.58) (width 0.25) (layer B.Cu) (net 7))
 (segment (start 72.27 47.58) (end 72.39 47.7) (width 0.25) (layer B.Cu) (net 7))
 (segment (start 70.45 136.71) (end 69.85 136.71) (width 0.25) (layer B.Cu) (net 8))
 (segment (start 74.92746 67.31) (end 74.93 67.30746) (width 0.25) (layer F.Cu) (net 8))
 (segment (start 71.47 67.31) (end 74.92746 67.31) (width 0.25) (layer F.Cu) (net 8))
 (segment (start 71.75 134.81) (end 72.35 134.81) (width 0.25) (layer F.Cu) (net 8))
 (segment (start 69.85 136.71) (end 71.75 134.81) (width 0.25) (layer F.Cu) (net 8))
 (segment (start 73.250008 133.710164) (end 74.050007 132.910165) (width 0.25) (layer F.Cu) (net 8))
 (segment (start 74.879583 133.35) (end 73.66 133.35) (width 0.25) (layer F.Cu) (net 8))
 (segment (start 77.075011 131.154572) (end 74.879583 133.35) (width 0.25) (layer F.Cu) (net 8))
 (segment (start 77.075011 69.452471) (end 77.075011 131.154572) (width 0.25) (layer F.Cu) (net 8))
 (segment (start 74.93 67.30746) (end 77.075011 69.452471) (width 0.25) (layer F.Cu) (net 8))
 (segment (start 68.06746 67.30746) (end 68.07 67.31) (width 0.25) (layer F.Cu) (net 9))
 (segment (start 64.77 67.30746) (end 68.06746 67.30746) (width 0.25) (layer F.Cu) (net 9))
 (segment (start 74.77 51.56) (end 74.77 51.435) (width 0.25) (layer B.Cu) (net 9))
 (segment (start 64.77 67.30746) (end 64.77 66.05797) (width 0.25) (layer B.Cu) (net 9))
 (segment (start 74.77 52.88438) (end 72.39 55.26438) (width 0.25) (layer B.Cu) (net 9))
 (segment (start 72.39 55.26438) (end 72.39 58.42) (width 0.25) (layer B.Cu) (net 9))
 (segment (start 64.77 66.05797) (end 72.39 58.43797) (width 0.25) (layer B.Cu) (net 9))
 (segment (start 74.505001 141.325001) (end 74.2225 141.0425) (width 0.25) (layer F.Cu) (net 9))
 (segment (start 75.015001 141.325001) (end 74.505001 141.325001) (width 0.25) (layer F.Cu) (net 9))
 (segment (start 74.380001 141.200001) (end 74.2225 141.0425) (width 0.25) (layer F.Cu) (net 9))
 (segment (start 75.015001 141.200001) (end 75.015001 141.325001) (width 0.25) (layer F.Cu) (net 9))
 (segment (start 64.77 67.30746) (end 64.77 68.55695) (width 0.25) (layer F.Cu) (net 9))
 (segment (start 64.77 68.55695) (end 63.174999 70.151951) (width 0.25) (layer F.Cu) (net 9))
 (segment (start 63.074999 134.648001) (end 63.273499 134.846501) (width 0.25) (layer F.Cu) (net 9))
 (segment (start 63.074999 72.338157) (end 63.074999 134.648001) (width 0.25) (layer F.Cu) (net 9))
 (segment (start 63.174999 72.238157) (end 63.074999 72.338157) (width 0.25) (layer F.Cu) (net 9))
 (segment (start 63.174999 70.151951) (end 63.174999 72.238157) (width 0.25) (layer F.Cu) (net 9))
 (segment (start 63.174999 134.748001) (end 63.273499 134.846501) (width 0.25) (layer F.Cu) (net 9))
 (segment (start 63.273499 134.846501) (end 66.929498 138.5025) (width 0.25) (layer F.Cu) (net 9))
 (segment (start 73.4175 138.5025) (end 70.4125 138.5025) (width 0.25) (layer F.Cu) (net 9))
 (segment (start 75.015001 140.100001) (end 73.4175 138.5025) (width 0.25) (layer F.Cu) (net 9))
 (segment (start 75.015001 141.325001) (end 75.015001 140.100001) (width 0.25) (layer F.Cu) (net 9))
 (segment (start 66.929498 138.5025) (end 70.4125 138.5025) (width 0.25) (layer F.Cu) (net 9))
 (segment (start 70.4125 138.5025) (end 71.6825 138.5025) (width 0.25) (layer F.Cu) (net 9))
 (segment (start 74.77 52.88438) (end 74.77 46.355) (width 0.25) (layer B.Cu) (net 9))
 (segment (start 65.749999 80.370001) (end 64.85 81.27) (width 0.25) (layer F.Cu) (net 1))
 (segment (start 65.970001 75.536813) (end 65.970001 80.149999) (width 0.25) (layer F.Cu) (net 1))
 (segment (start 65.970001 80.149999) (end 65.749999 80.370001) (width 0.25) (layer F.Cu) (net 1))
 (segment (start 67.311824 74.19499) (end 65.970001 75.536813) (width 0.25) (layer F.Cu) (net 1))
 (segment (start 73.250008 74.550926) (end 72.894072 74.19499) (width 0.25) (layer F.Cu) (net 1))
 (segment (start 73.250008 75.470164) (end 73.250008 74.550926) (width 0.25) (layer F.Cu) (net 1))
 (segment (start 65.668372 52.333372) (end 64.77 51.435) (width 0.25) (layer F.Cu) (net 1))
 (segment (start 70.38499 74.19499) (end 67.311824 74.19499) (width 0.25) (layer F.Cu) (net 1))
 (segment (start 72.894072 74.19499) (end 70.38499 74.19499) (width 0.25) (layer F.Cu) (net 1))
 (segment (start 64.77 51.435) (end 64.77 46.355) (width 0.25) (layer F.Cu) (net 1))
 (segment (start 65.749999 98.150001) (end 64.85 99.05) (width 0.25) (layer F.Cu) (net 1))
 (segment (start 66.04 97.86) (end 65.749999 98.150001) (width 0.25) (layer F.Cu) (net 1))
 (segment (start 66.04 93.246814) (end 66.04 97.86) (width 0.25) (layer F.Cu) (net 1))
 (segment (start 67.311824 91.97499) (end 66.04 93.246814) (width 0.25) (layer F.Cu) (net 1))
 (segment (start 72.894072 91.97499) (end 67.311824 91.97499) (width 0.25) (layer F.Cu) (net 1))
 (segment (start 73.250008 92.330926) (end 72.894072 91.97499) (width 0.25) (layer F.Cu) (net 1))
 (segment (start 73.250008 93.250164) (end 73.250008 92.330926) (width 0.25) (layer F.Cu) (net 1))
 (segment (start 66.04 115.64) (end 65.749999 115.930001) (width 0.25) (layer F.Cu) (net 1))
 (segment (start 66.04 111.026814) (end 66.04 115.64) (width 0.25) (layer F.Cu) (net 1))
 (segment (start 67.311824 109.75499) (end 66.04 111.026814) (width 0.25) (layer F.Cu) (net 1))
 (segment (start 72.894072 109.75499) (end 67.311824 109.75499) (width 0.25) (layer F.Cu) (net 1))
 (segment (start 73.250008 110.110926) (end 72.894072 109.75499) (width 0.25) (layer F.Cu) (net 1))
 (segment (start 65.749999 115.930001) (end 64.85 116.83) (width 0.25) (layer F.Cu) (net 1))
 (segment (start 73.250008 111.030164) (end 73.250008 110.110926) (width 0.25) (layer F.Cu) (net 1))
 (segment (start 67.311824 102.784616) (end 67.311824 109.75499) (width 0.25) (layer F.Cu) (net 1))
 (segment (start 64.85 100.322792) (end 67.311824 102.784616) (width 0.25) (layer F.Cu) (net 1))
 (segment (start 64.85 99.05) (end 64.85 100.322792) (width 0.25) (layer F.Cu) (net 1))
 (segment (start 67.311824 85.004616) (end 67.311824 91.97499) (width 0.25) (layer F.Cu) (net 1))
 (segment (start 64.85 82.542792) (end 67.311824 85.004616) (width 0.25) (layer F.Cu) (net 1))
 (segment (start 64.85 81.27) (end 64.85 82.542792) (width 0.25) (layer F.Cu) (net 1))
 (segment (start 65.749999 133.710001) (end 64.85 134.61) (width 0.25) (layer F.Cu) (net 1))
 (segment (start 66.04 133.42) (end 65.749999 133.710001) (width 0.25) (layer F.Cu) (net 1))
 (segment (start 66.04 128.806814) (end 66.04 133.42) (width 0.25) (layer F.Cu) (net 1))
 (segment (start 67.311824 127.53499) (end 66.04 128.806814) (width 0.25) (layer F.Cu) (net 1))
 (segment (start 73.250008 127.890926) (end 72.894072 127.53499) (width 0.25) (layer F.Cu) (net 1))
 (segment (start 72.894072 127.53499) (end 67.311824 127.53499) (width 0.25) (layer F.Cu) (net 1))
 (segment (start 73.250008 128.810164) (end 73.250008 127.890926) (width 0.25) (layer F.Cu) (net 1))
 (segment (start 67.311824 120.564616) (end 67.311824 127.53499) (width 0.25) (layer F.Cu) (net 1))
 (segment (start 64.85 118.102792) (end 67.311824 120.564616) (width 0.25) (layer F.Cu) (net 1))
 (segment (start 64.85 116.83) (end 64.85 118.102792) (width 0.25) (layer F.Cu) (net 1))
 (segment (start 65.015001 134.775001) (end 64.85 134.61) (width 0.25) (layer B.Cu) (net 1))
 (segment (start 65.015001 141.960001) (end 65.015001 134.775001) (width 0.25) (layer B.Cu) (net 1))
 (segment (start 69.85 74.19499) (end 69.85 73.66) (width 0.25) (layer F.Cu) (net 1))
 (segment (start 69.85 53.975) (end 69.85 74.19499) (width 0.25) (layer F.Cu) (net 1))
 (segment (start 64.77 51.435) (end 67.31 53.975) (width 0.25) (layer F.Cu) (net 1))
 (segment (start 67.31 53.975) (end 69.85 53.975) (width 0.25) (layer F.Cu) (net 1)))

